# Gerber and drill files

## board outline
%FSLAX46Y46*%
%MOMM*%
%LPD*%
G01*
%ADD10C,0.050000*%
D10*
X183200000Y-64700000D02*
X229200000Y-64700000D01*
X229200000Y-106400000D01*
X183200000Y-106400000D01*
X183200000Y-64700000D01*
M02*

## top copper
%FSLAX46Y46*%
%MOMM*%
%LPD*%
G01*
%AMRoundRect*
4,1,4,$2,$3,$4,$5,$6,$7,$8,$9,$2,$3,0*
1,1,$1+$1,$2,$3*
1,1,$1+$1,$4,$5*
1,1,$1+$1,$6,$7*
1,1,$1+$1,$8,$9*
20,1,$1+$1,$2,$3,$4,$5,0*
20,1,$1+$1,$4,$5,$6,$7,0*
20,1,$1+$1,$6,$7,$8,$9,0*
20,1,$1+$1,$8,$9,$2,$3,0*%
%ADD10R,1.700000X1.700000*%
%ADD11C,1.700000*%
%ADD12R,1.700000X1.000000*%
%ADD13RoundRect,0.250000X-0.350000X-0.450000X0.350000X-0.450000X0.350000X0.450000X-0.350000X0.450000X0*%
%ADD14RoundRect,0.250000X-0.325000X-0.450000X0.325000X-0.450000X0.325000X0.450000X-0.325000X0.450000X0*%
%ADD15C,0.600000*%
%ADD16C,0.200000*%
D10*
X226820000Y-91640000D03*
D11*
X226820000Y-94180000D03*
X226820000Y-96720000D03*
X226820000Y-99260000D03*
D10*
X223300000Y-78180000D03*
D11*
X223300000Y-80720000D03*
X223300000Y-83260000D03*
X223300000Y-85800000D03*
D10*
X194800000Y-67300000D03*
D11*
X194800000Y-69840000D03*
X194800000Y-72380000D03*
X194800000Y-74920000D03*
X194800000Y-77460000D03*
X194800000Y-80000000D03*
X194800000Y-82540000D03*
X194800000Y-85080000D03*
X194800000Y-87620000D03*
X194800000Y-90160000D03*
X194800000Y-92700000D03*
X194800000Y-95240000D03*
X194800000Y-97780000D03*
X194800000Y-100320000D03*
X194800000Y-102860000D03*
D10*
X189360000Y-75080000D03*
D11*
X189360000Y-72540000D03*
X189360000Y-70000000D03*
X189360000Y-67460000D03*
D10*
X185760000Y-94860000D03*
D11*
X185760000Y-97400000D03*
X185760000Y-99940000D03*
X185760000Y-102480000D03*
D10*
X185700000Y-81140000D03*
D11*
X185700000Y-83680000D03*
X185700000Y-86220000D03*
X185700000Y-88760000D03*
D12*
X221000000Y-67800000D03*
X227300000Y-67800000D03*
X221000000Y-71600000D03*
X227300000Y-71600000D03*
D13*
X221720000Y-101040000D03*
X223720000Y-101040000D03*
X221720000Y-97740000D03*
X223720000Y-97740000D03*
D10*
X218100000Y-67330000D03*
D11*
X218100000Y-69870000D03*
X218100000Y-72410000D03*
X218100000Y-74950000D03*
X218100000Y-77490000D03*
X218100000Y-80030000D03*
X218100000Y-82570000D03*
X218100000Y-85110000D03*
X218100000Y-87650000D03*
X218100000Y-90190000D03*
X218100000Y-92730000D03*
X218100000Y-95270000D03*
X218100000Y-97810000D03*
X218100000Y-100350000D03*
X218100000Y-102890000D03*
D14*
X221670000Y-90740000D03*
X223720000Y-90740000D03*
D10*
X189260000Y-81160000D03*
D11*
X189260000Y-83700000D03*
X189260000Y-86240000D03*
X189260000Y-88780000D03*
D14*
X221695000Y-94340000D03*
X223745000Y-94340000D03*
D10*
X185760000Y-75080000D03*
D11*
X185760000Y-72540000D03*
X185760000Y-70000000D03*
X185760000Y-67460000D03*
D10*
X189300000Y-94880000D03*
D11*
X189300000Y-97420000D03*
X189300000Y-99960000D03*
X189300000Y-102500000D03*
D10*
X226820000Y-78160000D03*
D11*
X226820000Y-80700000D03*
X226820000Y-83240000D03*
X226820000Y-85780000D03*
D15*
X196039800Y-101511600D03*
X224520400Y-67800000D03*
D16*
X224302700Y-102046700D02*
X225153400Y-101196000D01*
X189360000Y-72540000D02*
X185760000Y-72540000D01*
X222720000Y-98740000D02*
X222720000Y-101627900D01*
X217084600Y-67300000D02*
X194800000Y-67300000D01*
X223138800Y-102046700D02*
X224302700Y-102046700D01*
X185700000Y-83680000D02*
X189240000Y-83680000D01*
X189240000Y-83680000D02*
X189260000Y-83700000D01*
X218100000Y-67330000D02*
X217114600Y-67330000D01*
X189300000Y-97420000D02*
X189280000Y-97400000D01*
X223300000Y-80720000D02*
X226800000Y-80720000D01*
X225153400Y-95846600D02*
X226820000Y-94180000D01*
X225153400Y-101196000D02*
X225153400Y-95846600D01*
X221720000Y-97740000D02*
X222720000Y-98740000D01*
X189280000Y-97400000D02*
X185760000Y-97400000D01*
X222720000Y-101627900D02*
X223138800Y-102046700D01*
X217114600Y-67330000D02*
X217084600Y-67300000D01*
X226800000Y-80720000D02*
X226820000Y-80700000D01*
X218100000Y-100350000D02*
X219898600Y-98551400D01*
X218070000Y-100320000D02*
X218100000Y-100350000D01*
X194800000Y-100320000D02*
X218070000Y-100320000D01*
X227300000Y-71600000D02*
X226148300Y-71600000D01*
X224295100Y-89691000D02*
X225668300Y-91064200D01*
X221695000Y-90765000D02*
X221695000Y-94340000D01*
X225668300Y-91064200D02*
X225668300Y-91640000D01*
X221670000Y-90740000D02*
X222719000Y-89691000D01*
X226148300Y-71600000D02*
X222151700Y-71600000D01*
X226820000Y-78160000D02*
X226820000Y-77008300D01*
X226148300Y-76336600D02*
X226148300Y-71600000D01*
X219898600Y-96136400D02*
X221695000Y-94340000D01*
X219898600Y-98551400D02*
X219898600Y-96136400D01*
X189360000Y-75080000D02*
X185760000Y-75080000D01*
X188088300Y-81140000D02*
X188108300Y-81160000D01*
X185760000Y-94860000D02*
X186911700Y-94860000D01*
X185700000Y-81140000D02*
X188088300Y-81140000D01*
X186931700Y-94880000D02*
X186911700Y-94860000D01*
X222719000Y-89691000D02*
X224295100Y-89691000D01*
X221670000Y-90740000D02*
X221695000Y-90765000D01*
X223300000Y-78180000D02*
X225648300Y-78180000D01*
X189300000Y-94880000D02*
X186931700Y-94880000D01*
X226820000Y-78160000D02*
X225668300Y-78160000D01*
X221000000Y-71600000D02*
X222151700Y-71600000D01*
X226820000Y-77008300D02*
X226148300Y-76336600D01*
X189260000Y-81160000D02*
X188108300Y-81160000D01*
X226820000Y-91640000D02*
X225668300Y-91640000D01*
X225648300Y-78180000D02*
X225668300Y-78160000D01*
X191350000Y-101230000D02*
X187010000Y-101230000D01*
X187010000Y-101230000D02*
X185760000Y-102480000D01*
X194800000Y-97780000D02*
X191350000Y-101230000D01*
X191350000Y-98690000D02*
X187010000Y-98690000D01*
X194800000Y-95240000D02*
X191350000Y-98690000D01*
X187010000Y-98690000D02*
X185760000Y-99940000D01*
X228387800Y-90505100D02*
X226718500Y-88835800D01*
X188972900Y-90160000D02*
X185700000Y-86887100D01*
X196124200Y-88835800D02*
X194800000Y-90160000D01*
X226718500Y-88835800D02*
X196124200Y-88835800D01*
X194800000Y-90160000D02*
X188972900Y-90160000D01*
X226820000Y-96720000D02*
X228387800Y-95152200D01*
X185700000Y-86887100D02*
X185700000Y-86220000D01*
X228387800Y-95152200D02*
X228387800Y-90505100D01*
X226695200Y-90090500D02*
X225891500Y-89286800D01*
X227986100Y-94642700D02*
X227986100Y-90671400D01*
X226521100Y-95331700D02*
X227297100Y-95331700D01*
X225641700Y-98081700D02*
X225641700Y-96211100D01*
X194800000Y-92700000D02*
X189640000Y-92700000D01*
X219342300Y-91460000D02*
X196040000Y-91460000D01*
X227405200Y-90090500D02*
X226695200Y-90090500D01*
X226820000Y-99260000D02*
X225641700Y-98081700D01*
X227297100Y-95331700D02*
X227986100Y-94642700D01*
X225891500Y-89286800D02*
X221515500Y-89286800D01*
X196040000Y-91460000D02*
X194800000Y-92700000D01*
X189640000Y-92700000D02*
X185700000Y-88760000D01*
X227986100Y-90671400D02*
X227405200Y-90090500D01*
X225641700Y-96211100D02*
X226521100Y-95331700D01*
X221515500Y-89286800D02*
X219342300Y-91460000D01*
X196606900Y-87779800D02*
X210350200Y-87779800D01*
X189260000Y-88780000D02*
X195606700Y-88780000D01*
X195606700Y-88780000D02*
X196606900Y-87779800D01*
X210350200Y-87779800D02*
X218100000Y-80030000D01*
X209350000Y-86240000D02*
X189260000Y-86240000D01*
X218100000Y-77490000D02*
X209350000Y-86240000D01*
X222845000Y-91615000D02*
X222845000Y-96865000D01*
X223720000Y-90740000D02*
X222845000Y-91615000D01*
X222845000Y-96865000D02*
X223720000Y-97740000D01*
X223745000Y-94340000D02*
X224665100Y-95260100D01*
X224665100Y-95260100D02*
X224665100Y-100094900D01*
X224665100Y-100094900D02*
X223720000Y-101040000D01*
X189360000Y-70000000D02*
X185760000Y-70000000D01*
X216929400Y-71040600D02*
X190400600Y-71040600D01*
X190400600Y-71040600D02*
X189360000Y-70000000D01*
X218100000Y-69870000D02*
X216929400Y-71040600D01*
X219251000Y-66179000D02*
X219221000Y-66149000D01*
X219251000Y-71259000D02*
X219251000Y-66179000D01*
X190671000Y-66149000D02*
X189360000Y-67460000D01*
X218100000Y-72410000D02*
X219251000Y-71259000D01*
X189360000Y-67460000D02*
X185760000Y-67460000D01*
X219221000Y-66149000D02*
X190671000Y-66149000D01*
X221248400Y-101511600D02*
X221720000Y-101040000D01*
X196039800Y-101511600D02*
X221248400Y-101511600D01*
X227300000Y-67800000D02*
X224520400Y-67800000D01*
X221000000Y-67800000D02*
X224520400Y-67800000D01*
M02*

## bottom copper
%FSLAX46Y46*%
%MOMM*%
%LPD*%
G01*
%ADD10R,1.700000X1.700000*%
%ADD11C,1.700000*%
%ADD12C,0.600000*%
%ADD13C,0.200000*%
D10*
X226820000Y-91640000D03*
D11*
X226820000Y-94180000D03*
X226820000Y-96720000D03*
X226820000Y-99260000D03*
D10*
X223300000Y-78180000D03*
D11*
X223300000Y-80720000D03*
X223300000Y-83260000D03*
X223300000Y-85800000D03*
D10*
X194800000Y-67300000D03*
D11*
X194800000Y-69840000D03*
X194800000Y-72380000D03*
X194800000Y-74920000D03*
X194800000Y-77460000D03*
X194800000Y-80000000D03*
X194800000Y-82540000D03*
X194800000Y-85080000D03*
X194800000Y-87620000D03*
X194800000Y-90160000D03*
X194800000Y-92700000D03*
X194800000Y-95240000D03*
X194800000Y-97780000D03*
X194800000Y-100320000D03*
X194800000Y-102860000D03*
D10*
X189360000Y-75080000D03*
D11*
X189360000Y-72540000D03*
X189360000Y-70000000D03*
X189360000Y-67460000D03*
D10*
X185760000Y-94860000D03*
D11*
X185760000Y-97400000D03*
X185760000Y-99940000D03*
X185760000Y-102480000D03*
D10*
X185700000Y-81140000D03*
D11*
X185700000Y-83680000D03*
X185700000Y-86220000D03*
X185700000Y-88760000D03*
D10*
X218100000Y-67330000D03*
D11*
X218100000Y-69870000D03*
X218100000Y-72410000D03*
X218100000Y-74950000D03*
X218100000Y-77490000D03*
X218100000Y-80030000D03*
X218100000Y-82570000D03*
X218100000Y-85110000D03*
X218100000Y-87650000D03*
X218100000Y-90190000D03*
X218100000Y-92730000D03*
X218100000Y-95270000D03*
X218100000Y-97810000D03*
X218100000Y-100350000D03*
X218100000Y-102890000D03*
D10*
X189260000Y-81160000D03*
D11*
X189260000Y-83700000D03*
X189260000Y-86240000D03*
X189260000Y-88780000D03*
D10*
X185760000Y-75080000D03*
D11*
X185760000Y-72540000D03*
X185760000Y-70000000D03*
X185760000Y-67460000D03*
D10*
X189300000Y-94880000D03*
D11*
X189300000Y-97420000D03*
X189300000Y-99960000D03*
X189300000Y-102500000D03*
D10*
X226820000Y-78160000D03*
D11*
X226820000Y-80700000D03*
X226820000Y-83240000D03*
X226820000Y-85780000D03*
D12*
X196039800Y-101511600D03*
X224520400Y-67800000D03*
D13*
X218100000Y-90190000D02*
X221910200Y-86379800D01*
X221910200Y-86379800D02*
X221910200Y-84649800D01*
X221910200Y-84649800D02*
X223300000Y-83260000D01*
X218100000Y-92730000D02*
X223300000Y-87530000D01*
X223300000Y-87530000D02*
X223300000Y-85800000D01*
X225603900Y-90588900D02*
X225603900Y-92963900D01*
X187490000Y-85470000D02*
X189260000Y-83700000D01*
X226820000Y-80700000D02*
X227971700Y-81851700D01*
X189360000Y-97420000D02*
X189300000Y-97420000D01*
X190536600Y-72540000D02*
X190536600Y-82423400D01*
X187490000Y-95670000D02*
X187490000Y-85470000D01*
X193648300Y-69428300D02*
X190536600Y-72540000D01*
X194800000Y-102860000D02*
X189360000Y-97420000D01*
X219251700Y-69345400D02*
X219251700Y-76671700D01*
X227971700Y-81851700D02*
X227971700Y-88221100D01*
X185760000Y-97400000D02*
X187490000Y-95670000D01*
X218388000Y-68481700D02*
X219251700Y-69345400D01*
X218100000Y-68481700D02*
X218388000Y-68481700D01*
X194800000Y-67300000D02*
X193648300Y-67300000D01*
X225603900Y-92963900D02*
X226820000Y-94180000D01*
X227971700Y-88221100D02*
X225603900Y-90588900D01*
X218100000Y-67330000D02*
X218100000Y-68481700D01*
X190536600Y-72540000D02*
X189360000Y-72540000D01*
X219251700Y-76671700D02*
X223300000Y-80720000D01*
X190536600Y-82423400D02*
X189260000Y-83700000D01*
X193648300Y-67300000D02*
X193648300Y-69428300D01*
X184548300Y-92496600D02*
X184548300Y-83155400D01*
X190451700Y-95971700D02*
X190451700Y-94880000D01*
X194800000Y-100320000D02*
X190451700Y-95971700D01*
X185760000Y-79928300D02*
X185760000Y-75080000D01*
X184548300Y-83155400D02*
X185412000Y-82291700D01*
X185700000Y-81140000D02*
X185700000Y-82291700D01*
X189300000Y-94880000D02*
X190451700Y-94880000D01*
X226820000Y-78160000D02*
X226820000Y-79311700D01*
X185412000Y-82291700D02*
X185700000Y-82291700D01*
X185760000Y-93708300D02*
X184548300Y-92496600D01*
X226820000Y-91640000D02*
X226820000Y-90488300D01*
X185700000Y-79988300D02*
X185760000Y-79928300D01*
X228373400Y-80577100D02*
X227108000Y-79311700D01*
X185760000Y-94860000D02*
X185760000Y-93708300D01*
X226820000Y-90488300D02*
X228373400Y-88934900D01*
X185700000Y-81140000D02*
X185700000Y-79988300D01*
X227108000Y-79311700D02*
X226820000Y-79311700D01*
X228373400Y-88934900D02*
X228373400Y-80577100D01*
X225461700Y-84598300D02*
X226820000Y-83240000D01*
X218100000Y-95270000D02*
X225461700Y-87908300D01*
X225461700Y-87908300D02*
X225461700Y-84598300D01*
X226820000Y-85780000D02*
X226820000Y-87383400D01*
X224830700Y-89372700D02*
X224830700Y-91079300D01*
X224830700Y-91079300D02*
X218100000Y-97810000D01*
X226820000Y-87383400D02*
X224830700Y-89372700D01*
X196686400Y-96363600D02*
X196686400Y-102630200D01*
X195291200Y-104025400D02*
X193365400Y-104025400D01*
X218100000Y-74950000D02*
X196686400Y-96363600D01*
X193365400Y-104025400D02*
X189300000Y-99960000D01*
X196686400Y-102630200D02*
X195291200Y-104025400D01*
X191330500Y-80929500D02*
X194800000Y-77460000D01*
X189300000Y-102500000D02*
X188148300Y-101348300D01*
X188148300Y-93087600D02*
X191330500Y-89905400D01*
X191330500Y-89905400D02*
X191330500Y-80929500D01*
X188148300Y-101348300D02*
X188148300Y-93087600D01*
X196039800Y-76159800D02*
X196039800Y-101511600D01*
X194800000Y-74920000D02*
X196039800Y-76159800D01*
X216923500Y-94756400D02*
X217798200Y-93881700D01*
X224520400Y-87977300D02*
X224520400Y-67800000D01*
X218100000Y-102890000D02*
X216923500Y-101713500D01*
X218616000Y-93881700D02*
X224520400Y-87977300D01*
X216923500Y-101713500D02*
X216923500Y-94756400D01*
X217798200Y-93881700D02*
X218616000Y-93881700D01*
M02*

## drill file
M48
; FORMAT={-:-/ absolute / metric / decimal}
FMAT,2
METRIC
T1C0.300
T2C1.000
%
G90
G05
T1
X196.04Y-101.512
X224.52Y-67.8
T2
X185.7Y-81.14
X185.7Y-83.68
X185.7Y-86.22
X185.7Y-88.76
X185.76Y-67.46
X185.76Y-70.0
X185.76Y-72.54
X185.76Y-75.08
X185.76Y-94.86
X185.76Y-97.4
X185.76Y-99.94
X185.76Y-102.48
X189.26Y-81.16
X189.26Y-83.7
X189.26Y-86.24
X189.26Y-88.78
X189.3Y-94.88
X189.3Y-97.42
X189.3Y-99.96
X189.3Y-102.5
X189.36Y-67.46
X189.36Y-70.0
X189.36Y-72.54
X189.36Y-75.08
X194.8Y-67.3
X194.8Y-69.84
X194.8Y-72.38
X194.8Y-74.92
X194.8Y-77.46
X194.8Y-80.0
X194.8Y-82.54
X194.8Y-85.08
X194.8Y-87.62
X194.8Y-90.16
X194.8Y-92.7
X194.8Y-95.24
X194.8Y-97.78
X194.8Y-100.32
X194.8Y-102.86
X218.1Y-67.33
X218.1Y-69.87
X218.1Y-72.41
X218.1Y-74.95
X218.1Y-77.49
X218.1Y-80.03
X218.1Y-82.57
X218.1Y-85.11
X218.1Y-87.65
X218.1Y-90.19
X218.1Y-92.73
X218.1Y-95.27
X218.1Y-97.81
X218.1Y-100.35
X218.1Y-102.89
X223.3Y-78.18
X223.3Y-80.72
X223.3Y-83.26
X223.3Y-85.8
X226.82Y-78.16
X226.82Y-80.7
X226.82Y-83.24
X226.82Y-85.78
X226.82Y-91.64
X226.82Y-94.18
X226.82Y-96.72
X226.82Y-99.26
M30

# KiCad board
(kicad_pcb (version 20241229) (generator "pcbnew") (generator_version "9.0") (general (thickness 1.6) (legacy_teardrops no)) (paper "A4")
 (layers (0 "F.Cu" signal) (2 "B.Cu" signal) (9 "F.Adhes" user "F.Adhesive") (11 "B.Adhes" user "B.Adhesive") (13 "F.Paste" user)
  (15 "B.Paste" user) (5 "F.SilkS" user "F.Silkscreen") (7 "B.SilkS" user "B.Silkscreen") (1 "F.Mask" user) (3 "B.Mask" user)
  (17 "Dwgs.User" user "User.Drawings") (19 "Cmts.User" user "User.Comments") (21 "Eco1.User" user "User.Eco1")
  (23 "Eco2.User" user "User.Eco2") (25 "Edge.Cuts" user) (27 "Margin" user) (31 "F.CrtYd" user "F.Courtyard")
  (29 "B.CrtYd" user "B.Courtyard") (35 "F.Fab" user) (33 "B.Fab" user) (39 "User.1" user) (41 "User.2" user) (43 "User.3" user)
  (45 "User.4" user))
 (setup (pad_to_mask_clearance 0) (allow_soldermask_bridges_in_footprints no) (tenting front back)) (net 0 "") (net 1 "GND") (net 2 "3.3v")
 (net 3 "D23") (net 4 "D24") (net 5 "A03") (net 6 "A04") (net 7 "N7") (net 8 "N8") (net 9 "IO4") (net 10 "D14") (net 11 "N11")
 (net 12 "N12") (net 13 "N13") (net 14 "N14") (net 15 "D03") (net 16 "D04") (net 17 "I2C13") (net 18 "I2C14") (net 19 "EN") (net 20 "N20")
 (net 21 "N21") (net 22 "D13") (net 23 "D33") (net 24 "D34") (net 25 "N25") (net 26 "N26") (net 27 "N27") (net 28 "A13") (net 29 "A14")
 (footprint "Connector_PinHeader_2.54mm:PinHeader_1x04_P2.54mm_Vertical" (layer "F.Cu") (at 226.82 91.64)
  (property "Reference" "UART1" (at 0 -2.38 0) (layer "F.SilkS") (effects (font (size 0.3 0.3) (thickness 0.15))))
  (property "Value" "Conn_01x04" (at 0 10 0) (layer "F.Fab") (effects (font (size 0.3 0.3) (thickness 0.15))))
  (pad "1" thru_hole rect (at 0 0) (size 1.7 1.7) (drill 1) (layers "*.Cu" "*.Mask") (remove_unused_layers no) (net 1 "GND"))
  (pad "2" thru_hole circle (at 0 2.54) (size 1.7 1.7) (drill 1) (layers "*.Cu" "*.Mask") (remove_unused_layers no) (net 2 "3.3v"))
  (pad "3" thru_hole circle (at 0 5.08) (size 1.7 1.7) (drill 1) (layers "*.Cu" "*.Mask") (remove_unused_layers no) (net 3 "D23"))
  (pad "4" thru_hole circle (at 0 7.62) (size 1.7 1.7) (drill 1) (layers "*.Cu" "*.Mask") (remove_unused_layers no) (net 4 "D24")))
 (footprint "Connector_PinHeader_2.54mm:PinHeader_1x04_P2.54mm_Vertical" (layer "F.Cu") (at 223.3 78.18)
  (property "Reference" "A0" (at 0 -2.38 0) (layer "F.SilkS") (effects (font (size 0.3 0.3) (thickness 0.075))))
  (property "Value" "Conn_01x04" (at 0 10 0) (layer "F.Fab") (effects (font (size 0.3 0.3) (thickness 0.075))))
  (pad "1" thru_hole rect (at 0 0) (size 1.7 1.7) (drill 1) (layers "*.Cu" "*.Mask") (remove_unused_layers no) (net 1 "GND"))
  (pad "2" thru_hole circle (at 0 2.54) (size 1.7 1.7) (drill 1) (layers "*.Cu" "*.Mask") (remove_unused_layers no) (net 2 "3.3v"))
  (pad "3" thru_hole circle (at 0 5.08) (size 1.7 1.7) (drill 1) (layers "*.Cu" "*.Mask") (remove_unused_layers no) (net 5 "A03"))
  (pad "4" thru_hole circle (at 0 7.62) (size 1.7 1.7) (drill 1) (layers "*.Cu" "*.Mask") (remove_unused_layers no) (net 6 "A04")))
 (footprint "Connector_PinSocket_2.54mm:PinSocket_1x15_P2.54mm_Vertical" (layer "F.Cu") (at 194.8 67.3)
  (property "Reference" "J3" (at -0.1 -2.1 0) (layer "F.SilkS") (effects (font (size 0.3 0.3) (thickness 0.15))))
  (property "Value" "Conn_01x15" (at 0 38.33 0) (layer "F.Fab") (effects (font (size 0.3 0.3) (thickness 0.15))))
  (pad "1" thru_hole rect (at 0 0) (size 1.7 1.7) (drill 1) (layers "*.Cu" "*.Mask") (remove_unused_layers no) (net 2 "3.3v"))
  (pad "2" thru_hole circle (at 0 2.54) (size 1.7 1.7) (drill 1) (layers "*.Cu" "*.Mask") (remove_unused_layers no) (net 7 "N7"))
  (pad "3" thru_hole circle (at 0 5.08) (size 1.7 1.7) (drill 1) (layers "*.Cu" "*.Mask") (remove_unused_layers no) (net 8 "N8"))
  (pad "4" thru_hole circle (at 0 7.62) (size 1.7 1.7) (drill 1) (layers "*.Cu" "*.Mask") (remove_unused_layers no) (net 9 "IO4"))
  (pad "5" thru_hole circle (at 0 10.16) (size 1.7 1.7) (drill 1) (layers "*.Cu" "*.Mask") (remove_unused_layers no) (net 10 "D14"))
  (pad "6" thru_hole circle (at 0 12.7) (size 1.7 1.7) (drill 1) (layers "*.Cu" "*.Mask") (remove_unused_layers no) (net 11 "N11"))
  (pad "7" thru_hole circle (at 0 15.24) (size 1.7 1.7) (drill 1) (layers "*.Cu" "*.Mask") (remove_unused_layers no) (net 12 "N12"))
  (pad "8" thru_hole circle (at 0 17.78) (size 1.7 1.7) (drill 1) (layers "*.Cu" "*.Mask") (remove_unused_layers no) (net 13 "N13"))
  (pad "9" thru_hole circle (at 0 20.32) (size 1.7 1.7) (drill 1) (layers "*.Cu" "*.Mask") (remove_unused_layers no) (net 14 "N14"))
  (pad "10" thru_hole circle (at 0 22.86) (size 1.7 1.7) (drill 1) (layers "*.Cu" "*.Mask") (remove_unused_layers no) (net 3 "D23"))
  (pad "11" thru_hole circle (at 0 25.4) (size 1.7 1.7) (drill 1) (layers "*.Cu" "*.Mask") (remove_unused_layers no) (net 4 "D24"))
  (pad "12" thru_hole circle (at 0 27.94) (size 1.7 1.7) (drill 1) (layers "*.Cu" "*.Mask") (remove_unused_layers no) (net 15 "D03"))
  (pad "13" thru_hole circle (at 0 30.48) (size 1.7 1.7) (drill 1) (layers "*.Cu" "*.Mask") (remove_unused_layers no) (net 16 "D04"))
  (pad "14" thru_hole circle (at 0 33.02) (size 1.7 1.7) (drill 1) (layers "*.Cu" "*.Mask") (remove_unused_layers no) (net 1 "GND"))
  (pad "15" thru_hole circle (at 0 35.56) (size 1.7 1.7) (drill 1) (layers "*.Cu" "*.Mask") (remove_unused_layers no) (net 2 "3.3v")))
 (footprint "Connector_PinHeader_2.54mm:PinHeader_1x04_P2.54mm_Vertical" (layer "F.Cu") (at 189.36 75.08 180)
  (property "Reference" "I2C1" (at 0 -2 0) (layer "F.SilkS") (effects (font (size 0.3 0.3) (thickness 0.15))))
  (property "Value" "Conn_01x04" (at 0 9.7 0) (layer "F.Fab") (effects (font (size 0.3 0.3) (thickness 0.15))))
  (pad "1" thru_hole rect (at 0 0 180) (size 1.7 1.7) (drill 1) (layers "*.Cu" "*.Mask") (remove_unused_layers no) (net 1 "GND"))
  (pad "2" thru_hole circle (at 0 2.54 180) (size 1.7 1.7) (drill 1) (layers "*.Cu" "*.Mask") (remove_unused_layers no) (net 2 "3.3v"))
  (pad "3" thru_hole circle (at 0 5.08 180) (size 1.7 1.7) (drill 1) (layers "*.Cu" "*.Mask") (remove_unused_layers no) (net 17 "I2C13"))
  (pad "4" thru_hole circle (at 0 7.62 180) (size 1.7 1.7) (drill 1) (layers "*.Cu" "*.Mask") (remove_unused_layers no) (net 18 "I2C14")))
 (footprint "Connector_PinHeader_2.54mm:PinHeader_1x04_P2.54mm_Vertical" (layer "F.Cu") (at 185.76 94.86)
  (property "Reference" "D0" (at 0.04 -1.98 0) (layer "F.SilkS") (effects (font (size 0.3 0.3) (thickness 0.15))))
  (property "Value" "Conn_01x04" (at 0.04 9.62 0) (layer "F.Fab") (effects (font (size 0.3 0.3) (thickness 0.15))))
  (pad "1" thru_hole rect (at 0 0) (size 1.7 1.7) (drill 1) (layers "*.Cu" "*.Mask") (remove_unused_layers no) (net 1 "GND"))
  (pad "2" thru_hole circle (at 0 2.54) (size 1.7 1.7) (drill 1) (layers "*.Cu" "*.Mask") (remove_unused_layers no) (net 2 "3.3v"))
  (pad "3" thru_hole circle (at 0 5.08) (size 1.7 1.7) (drill 1) (layers "*.Cu" "*.Mask") (remove_unused_layers no) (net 15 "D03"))
  (pad "4" thru_hole circle (at 0 7.62) (size 1.7 1.7) (drill 1) (layers "*.Cu" "*.Mask") (remove_unused_layers no) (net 16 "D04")))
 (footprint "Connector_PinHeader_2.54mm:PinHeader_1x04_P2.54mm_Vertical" (layer "F.Cu") (at 185.7 81.14)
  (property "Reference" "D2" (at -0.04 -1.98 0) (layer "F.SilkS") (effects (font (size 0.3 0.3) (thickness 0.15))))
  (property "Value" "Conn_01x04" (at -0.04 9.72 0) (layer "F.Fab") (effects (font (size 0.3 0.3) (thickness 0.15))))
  (pad "1" thru_hole rect (at 0 0) (size 1.7 1.7) (drill 1) (layers "*.Cu" "*.Mask") (remove_unused_layers no) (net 1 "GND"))
  (pad "2" thru_hole circle (at 0 2.54) (size 1.7 1.7) (drill 1) (layers "*.Cu" "*.Mask") (remove_unused_layers no) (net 2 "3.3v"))
  (pad "3" thru_hole circle (at 0 5.08) (size 1.7 1.7) (drill 1) (layers "*.Cu" "*.Mask") (remove_unused_layers no) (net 3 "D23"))
  (pad "4" thru_hole circle (at 0 7.62) (size 1.7 1.7) (drill 1) (layers "*.Cu" "*.Mask") (remove_unused_layers no) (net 4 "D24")))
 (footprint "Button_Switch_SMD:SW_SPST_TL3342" (layer "F.Cu") (at 224.15 69.7)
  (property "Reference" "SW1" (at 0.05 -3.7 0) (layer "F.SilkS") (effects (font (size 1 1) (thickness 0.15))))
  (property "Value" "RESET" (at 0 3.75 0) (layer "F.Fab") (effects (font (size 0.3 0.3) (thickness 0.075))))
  (pad "1" smd rect (at -3.15 -1.9) (size 1.7 1) (layers "F.Cu" "F.Mask" "F.Paste") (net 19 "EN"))
  (pad "1" smd rect (at 3.15 -1.9) (size 1.7 1) (layers "F.Cu" "F.Mask" "F.Paste") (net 19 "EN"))
  (pad "2" smd rect (at -3.15 1.9) (size 1.7 1) (layers "F.Cu" "F.Mask" "F.Paste") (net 1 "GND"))
  (pad "2" smd rect (at 3.15 1.9) (size 1.7 1) (layers "F.Cu" "F.Mask" "F.Paste") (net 1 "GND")))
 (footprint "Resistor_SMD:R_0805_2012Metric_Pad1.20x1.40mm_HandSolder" (layer "F.Cu") (at 222.72 101.04)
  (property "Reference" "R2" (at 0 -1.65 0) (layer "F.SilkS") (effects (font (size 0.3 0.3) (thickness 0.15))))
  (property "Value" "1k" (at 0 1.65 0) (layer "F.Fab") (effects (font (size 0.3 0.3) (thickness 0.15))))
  (pad "1" smd roundrect (at -1 0) (size 1.2 1.4) (layers "F.Cu" "F.Mask" "F.Paste") (roundrect_rratio 0.208333) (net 9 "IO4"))
  (pad "2" smd roundrect (at 1 0) (size 1.2 1.4) (layers "F.Cu" "F.Mask" "F.Paste") (roundrect_rratio 0.208333) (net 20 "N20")))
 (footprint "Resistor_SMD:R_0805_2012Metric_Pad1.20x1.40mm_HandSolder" (layer "F.Cu") (at 222.72 97.74)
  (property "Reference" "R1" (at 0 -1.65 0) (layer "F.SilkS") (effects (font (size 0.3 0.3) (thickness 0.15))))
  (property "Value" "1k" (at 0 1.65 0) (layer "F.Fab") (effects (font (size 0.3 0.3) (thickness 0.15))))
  (pad "1" smd roundrect (at -1 0) (size 1.2 1.4) (layers "F.Cu" "F.Mask" "F.Paste") (roundrect_rratio 0.208333) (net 2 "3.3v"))
  (pad "2" smd roundrect (at 1 0) (size 1.2 1.4) (layers "F.Cu" "F.Mask" "F.Paste") (roundrect_rratio 0.208333) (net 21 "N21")))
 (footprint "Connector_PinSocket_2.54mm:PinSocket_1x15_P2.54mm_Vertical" (layer "F.Cu") (at 218.1 67.33)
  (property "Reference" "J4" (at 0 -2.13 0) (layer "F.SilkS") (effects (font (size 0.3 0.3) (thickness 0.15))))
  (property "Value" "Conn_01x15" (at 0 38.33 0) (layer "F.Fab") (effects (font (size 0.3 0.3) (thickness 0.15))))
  (pad "1" thru_hole rect (at 0 0) (size 1.7 1.7) (drill 1) (layers "*.Cu" "*.Mask") (remove_unused_layers no) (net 2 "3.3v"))
  (pad "2" thru_hole circle (at 0 2.54) (size 1.7 1.7) (drill 1) (layers "*.Cu" "*.Mask") (remove_unused_layers no) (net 17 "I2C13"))
  (pad "3" thru_hole circle (at 0 5.08) (size 1.7 1.7) (drill 1) (layers "*.Cu" "*.Mask") (remove_unused_layers no) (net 18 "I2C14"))
  (pad "4" thru_hole circle (at 0 7.62) (size 1.7 1.7) (drill 1) (layers "*.Cu" "*.Mask") (remove_unused_layers no) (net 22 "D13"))
  (pad "5" thru_hole circle (at 0 10.16) (size 1.7 1.7) (drill 1) (layers "*.Cu" "*.Mask") (remove_unused_layers no) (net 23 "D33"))
  (pad "6" thru_hole circle (at 0 12.7) (size 1.7 1.7) (drill 1) (layers "*.Cu" "*.Mask") (remove_unused_layers no) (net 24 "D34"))
  (pad "7" thru_hole circle (at 0 15.24) (size 1.7 1.7) (drill 1) (layers "*.Cu" "*.Mask") (remove_unused_layers no) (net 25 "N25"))
  (pad "8" thru_hole circle (at 0 17.78) (size 1.7 1.7) (drill 1) (layers "*.Cu" "*.Mask") (remove_unused_layers no) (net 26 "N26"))
  (pad "9" thru_hole circle (at 0 20.32) (size 1.7 1.7) (drill 1) (layers "*.Cu" "*.Mask") (remove_unused_layers no) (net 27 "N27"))
  (pad "10" thru_hole circle (at 0 22.86) (size 1.7 1.7) (drill 1) (layers "*.Cu" "*.Mask") (remove_unused_layers no) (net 5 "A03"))
  (pad "11" thru_hole circle (at 0 25.4) (size 1.7 1.7) (drill 1) (layers "*.Cu" "*.Mask") (remove_unused_layers no) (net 6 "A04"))
  (pad "12" thru_hole circle (at 0 27.94) (size 1.7 1.7) (drill 1) (layers "*.Cu" "*.Mask") (remove_unused_layers no) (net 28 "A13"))
  (pad "13" thru_hole circle (at 0 30.48) (size 1.7 1.7) (drill 1) (layers "*.Cu" "*.Mask") (remove_unused_layers no) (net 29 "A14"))
  (pad "14" thru_hole circle (at 0 33.02) (size 1.7 1.7) (drill 1) (layers "*.Cu" "*.Mask") (remove_unused_layers no) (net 1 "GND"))
  (pad "15" thru_hole circle (at 0 35.56) (size 1.7 1.7) (drill 1) (layers "*.Cu" "*.Mask") (remove_unused_layers no) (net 19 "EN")))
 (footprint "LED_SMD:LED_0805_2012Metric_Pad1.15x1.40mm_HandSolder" (layer "F.Cu") (at 222.695 90.74)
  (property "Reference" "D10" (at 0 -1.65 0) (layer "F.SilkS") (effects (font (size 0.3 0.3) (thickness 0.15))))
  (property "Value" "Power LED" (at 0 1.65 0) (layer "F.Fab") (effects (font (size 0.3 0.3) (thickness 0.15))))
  (pad "1" smd roundrect (at -1.025 0) (size 1.15 1.4) (layers "F.Cu" "F.Mask" "F.Paste") (roundrect_rratio 0.217391) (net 1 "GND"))
  (pad "2" smd roundrect (at 1.025 0) (size 1.15 1.4) (layers "F.Cu" "F.Mask" "F.Paste") (roundrect_rratio 0.217391) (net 21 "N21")))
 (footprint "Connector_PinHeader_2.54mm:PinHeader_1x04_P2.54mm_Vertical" (layer "F.Cu") (at 189.26 81.16)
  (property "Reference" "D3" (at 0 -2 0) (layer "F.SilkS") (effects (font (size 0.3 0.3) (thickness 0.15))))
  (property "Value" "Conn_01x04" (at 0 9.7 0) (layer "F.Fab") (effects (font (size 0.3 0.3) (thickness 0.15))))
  (pad "1" thru_hole rect (at 0 0) (size 1.7 1.7) (drill 1) (layers "*.Cu" "*.Mask") (remove_unused_layers no) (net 1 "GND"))
  (pad "2" thru_hole circle (at 0 2.54) (size 1.7 1.7) (drill 1) (layers "*.Cu" "*.Mask") (remove_unused_layers no) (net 2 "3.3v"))
  (pad "3" thru_hole circle (at 0 5.08) (size 1.7 1.7) (drill 1) (layers "*.Cu" "*.Mask") (remove_unused_layers no) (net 23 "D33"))
  (pad "4" thru_hole circle (at 0 7.62) (size 1.7 1.7) (drill 1) (layers "*.Cu" "*.Mask") (remove_unused_layers no) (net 24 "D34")))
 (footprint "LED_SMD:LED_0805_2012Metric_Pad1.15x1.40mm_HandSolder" (layer "F.Cu") (at 222.72 94.34)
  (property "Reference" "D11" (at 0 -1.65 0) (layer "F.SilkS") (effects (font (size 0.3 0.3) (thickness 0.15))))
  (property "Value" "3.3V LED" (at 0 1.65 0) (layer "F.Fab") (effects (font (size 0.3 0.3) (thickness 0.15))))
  (pad "1" smd roundrect (at -1.025 0) (size 1.15 1.4) (layers "F.Cu" "F.Mask" "F.Paste") (roundrect_rratio 0.217391) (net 1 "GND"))
  (pad "2" smd roundrect (at 1.025 0) (size 1.15 1.4) (layers "F.Cu" "F.Mask" "F.Paste") (roundrect_rratio 0.217391) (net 20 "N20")))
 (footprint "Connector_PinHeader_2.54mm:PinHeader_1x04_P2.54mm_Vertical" (layer "F.Cu") (at 185.76 75.08 180)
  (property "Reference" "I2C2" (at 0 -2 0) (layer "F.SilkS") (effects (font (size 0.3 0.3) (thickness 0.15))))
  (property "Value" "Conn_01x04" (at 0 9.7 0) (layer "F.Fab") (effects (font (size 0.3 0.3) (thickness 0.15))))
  (pad "1" thru_hole rect (at 0 0 180) (size 1.7 1.7) (drill 1) (layers "*.Cu" "*.Mask") (remove_unused_layers no) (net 1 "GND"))
  (pad "2" thru_hole circle (at 0 2.54 180) (size 1.7 1.7) (drill 1) (layers "*.Cu" "*.Mask") (remove_unused_layers no) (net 2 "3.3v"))
  (pad "3" thru_hole circle (at 0 5.08 180) (size 1.7 1.7) (drill 1) (layers "*.Cu" "*.Mask") (remove_unused_layers no) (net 17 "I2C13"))
  (pad "4" thru_hole circle (at 0 7.62 180) (size 1.7 1.7) (drill 1) (layers "*.Cu" "*.Mask") (remove_unused_layers no) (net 18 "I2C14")))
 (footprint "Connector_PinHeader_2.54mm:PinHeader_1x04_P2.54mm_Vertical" (layer "F.Cu") (at 189.3 94.88)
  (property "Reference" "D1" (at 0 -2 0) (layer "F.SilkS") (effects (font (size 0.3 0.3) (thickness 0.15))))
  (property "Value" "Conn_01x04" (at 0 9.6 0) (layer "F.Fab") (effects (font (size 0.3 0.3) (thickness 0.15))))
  (pad "1" thru_hole rect (at 0 0) (size 1.7 1.7) (drill 1) (layers "*.Cu" "*.Mask") (remove_unused_layers no) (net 1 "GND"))
  (pad "2" thru_hole circle (at 0 2.54) (size 1.7 1.7) (drill 1) (layers "*.Cu" "*.Mask") (remove_unused_layers no) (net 2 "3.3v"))
  (pad "3" thru_hole circle (at 0 5.08) (size 1.7 1.7) (drill 1) (layers "*.Cu" "*.Mask") (remove_unused_layers no) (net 22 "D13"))
  (pad "4" thru_hole circle (at 0 7.62) (size 1.7 1.7) (drill 1) (layers "*.Cu" "*.Mask") (remove_unused_layers no) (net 10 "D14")))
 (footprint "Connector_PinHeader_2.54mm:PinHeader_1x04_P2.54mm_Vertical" (layer "F.Cu") (at 226.82 78.16)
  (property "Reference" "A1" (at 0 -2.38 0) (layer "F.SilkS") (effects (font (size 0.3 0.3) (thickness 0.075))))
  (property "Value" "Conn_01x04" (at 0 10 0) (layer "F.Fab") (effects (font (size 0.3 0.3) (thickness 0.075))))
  (pad "1" thru_hole rect (at 0 0) (size 1.7 1.7) (drill 1) (layers "*.Cu" "*.Mask") (remove_unused_layers no) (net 1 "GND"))
  (pad "2" thru_hole circle (at 0 2.54) (size 1.7 1.7) (drill 1) (layers "*.Cu" "*.Mask") (remove_unused_layers no) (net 2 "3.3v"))
  (pad "3" thru_hole circle (at 0 5.08) (size 1.7 1.7) (drill 1) (layers "*.Cu" "*.Mask") (remove_unused_layers no) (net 28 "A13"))
  (pad "4" thru_hole circle (at 0 7.62) (size 1.7 1.7) (drill 1) (layers "*.Cu" "*.Mask") (remove_unused_layers no) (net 29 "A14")))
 (gr_rect (start 183.2 64.7) (end 229.2 106.4) (stroke (width 0.05) (type default)) (fill no) (layer "Edge.Cuts"))
 (segment (start 218.1 90.19) (end 221.9102 86.3798) (width 0.2) (layer "B.Cu") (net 5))
 (segment (start 221.9102 86.3798) (end 221.9102 84.6498) (width 0.2) (layer "B.Cu") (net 5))
 (segment (start 221.9102 84.6498) (end 223.3 83.26) (width 0.2) (layer "B.Cu") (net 5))
 (segment (start 218.1 92.73) (end 223.3 87.53) (width 0.2) (layer "B.Cu") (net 6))
 (segment (start 223.3 87.53) (end 223.3 85.8) (width 0.2) (layer "B.Cu") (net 6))
 (segment (start 224.3027 102.0467) (end 225.1534 101.196) (width 0.2) (layer "F.Cu") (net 2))
 (segment (start 189.36 72.54) (end 185.76 72.54) (width 0.2) (layer "F.Cu") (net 2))
 (segment (start 222.72 98.74) (end 222.72 101.6279) (width 0.2) (layer "F.Cu") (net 2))
 (segment (start 217.0846 67.3) (end 194.8 67.3) (width 0.2) (layer "F.Cu") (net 2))
 (segment (start 223.1388 102.0467) (end 224.3027 102.0467) (width 0.2) (layer "F.Cu") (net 2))
 (segment (start 185.7 83.68) (end 189.24 83.68) (width 0.2) (layer "F.Cu") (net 2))
 (segment (start 189.24 83.68) (end 189.26 83.7) (width 0.2) (layer "F.Cu") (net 2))
 (segment (start 218.1 67.33) (end 217.1146 67.33) (width 0.2) (layer "F.Cu") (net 2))
 (segment (start 189.3 97.42) (end 189.28 97.4) (width 0.2) (layer "F.Cu") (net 2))
 (segment (start 223.3 80.72) (end 226.8 80.72) (width 0.2) (layer "F.Cu") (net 2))
 (segment (start 225.1534 95.8466) (end 226.82 94.18) (width 0.2) (layer "F.Cu") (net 2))
 (segment (start 225.1534 101.196) (end 225.1534 95.8466) (width 0.2) (layer "F.Cu") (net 2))
 (segment (start 221.72 97.74) (end 222.72 98.74) (width 0.2) (layer "F.Cu") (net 2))
 (segment (start 189.28 97.4) (end 185.76 97.4) (width 0.2) (layer "F.Cu") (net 2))
 (segment (start 222.72 101.6279) (end 223.1388 102.0467) (width 0.2) (layer "F.Cu") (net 2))
 (segment (start 217.1146 67.33) (end 217.0846 67.3) (width 0.2) (layer "F.Cu") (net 2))
 (segment (start 226.8 80.72) (end 226.82 80.7) (width 0.2) (layer "F.Cu") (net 2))
 (segment (start 225.6039 90.5889) (end 225.6039 92.9639) (width 0.2) (layer "B.Cu") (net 2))
 (segment (start 187.49 85.47) (end 189.26 83.7) (width 0.2) (layer "B.Cu") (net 2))
 (segment (start 226.82 80.7) (end 227.9717 81.8517) (width 0.2) (layer "B.Cu") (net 2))
 (segment (start 189.36 97.42) (end 189.3 97.42) (width 0.2) (layer "B.Cu") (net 2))
 (segment (start 190.5366 72.54) (end 190.5366 82.4234) (width 0.2) (layer "B.Cu") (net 2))
 (segment (start 187.49 95.67) (end 187.49 85.47) (width 0.2) (layer "B.Cu") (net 2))
 (segment (start 193.6483 69.4283) (end 190.5366 72.54) (width 0.2) (layer "B.Cu") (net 2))
 (segment (start 194.8 102.86) (end 189.36 97.42) (width 0.2) (layer "B.Cu") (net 2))
 (segment (start 219.2517 69.3454) (end 219.2517 76.6717) (width 0.2) (layer "B.Cu") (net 2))
 (segment (start 227.9717 81.8517) (end 227.9717 88.2211) (width 0.2) (layer "B.Cu") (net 2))
 (segment (start 185.76 97.4) (end 187.49 95.67) (width 0.2) (layer "B.Cu") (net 2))
 (segment (start 218.388 68.4817) (end 219.2517 69.3454) (width 0.2) (layer "B.Cu") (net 2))
 (segment (start 218.1 68.4817) (end 218.388 68.4817) (width 0.2) (layer "B.Cu") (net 2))
 (segment (start 194.8 67.3) (end 193.6483 67.3) (width 0.2) (layer "B.Cu") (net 2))
 (segment (start 225.6039 92.9639) (end 226.82 94.18) (width 0.2) (layer "B.Cu") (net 2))
 (segment (start 227.9717 88.2211) (end 225.6039 90.5889) (width 0.2) (layer "B.Cu") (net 2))
 (segment (start 218.1 67.33) (end 218.1 68.4817) (width 0.2) (layer "B.Cu") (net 2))
 (segment (start 190.5366 72.54) (end 189.36 72.54) (width 0.2) (layer "B.Cu") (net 2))
 (segment (start 219.2517 76.6717) (end 223.3 80.72) (width 0.2) (layer "B.Cu") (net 2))
 (segment (start 190.5366 82.4234) (end 189.26 83.7) (width 0.2) (layer "B.Cu") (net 2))
 (segment (start 193.6483 67.3) (end 193.6483 69.4283) (width 0.2) (layer "B.Cu") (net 2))
 (segment (start 218.1 100.35) (end 219.8986 98.5514) (width 0.2) (layer "F.Cu") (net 1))
 (segment (start 218.07 100.32) (end 218.1 100.35) (width 0.2) (layer "F.Cu") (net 1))
 (segment (start 194.8 100.32) (end 218.07 100.32) (width 0.2) (layer "F.Cu") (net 1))
 (segment (start 227.3 71.6) (end 226.1483 71.6) (width 0.2) (layer "F.Cu") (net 1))
 (segment (start 224.2951 89.691) (end 225.6683 91.0642) (width 0.2) (layer "F.Cu") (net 1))
 (segment (start 221.695 90.765) (end 221.695 94.34) (width 0.2) (layer "F.Cu") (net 1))
 (segment (start 225.6683 91.0642) (end 225.6683 91.64) (width 0.2) (layer "F.Cu") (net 1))
 (segment (start 221.67 90.74) (end 222.719 89.691) (width 0.2) (layer "F.Cu") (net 1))
 (segment (start 226.1483 71.6) (end 222.1517 71.6) (width 0.2) (layer "F.Cu") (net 1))
 (segment (start 226.82 78.16) (end 226.82 77.0083) (width 0.2) (layer "F.Cu") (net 1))
 (segment (start 226.1483 76.3366) (end 226.1483 71.6) (width 0.2) (layer "F.Cu") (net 1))
 (segment (start 219.8986 96.1364) (end 221.695 94.34) (width 0.2) (layer "F.Cu") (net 1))
 (segment (start 219.8986 98.5514) (end 219.8986 96.1364) (width 0.2) (layer "F.Cu") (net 1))
 (segment (start 189.36 75.08) (end 185.76 75.08) (width 0.2) (layer "F.Cu") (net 1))
 (segment (start 188.0883 81.14) (end 188.1083 81.16) (width 0.2) (layer "F.Cu") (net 1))
 (segment (start 185.76 94.86) (end 186.9117 94.86) (width 0.2) (layer "F.Cu") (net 1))
 (segment (start 185.7 81.14) (end 188.0883 81.14) (width 0.2) (layer "F.Cu") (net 1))
 (segment (start 186.9317 94.88) (end 186.9117 94.86) (width 0.2) (layer "F.Cu") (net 1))
 (segment (start 222.719 89.691) (end 224.2951 89.691) (width 0.2) (layer "F.Cu") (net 1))
 (segment (start 221.67 90.74) (end 221.695 90.765) (width 0.2) (layer "F.Cu") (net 1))
 (segment (start 223.3 78.18) (end 225.6483 78.18) (width 0.2) (layer "F.Cu") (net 1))
 (segment (start 189.3 94.88) (end 186.9317 94.88) (width 0.2) (layer "F.Cu") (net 1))
 (segment (start 226.82 78.16) (end 225.6683 78.16) (width 0.2) (layer "F.Cu") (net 1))
 (segment (start 221 71.6) (end 222.1517 71.6) (width 0.2) (layer "F.Cu") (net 1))
 (segment (start 226.82 77.0083) (end 226.1483 76.3366) (width 0.2) (layer "F.Cu") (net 1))
 (segment (start 189.26 81.16) (end 188.1083 81.16) (width 0.2) (layer "F.Cu") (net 1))
 (segment (start 226.82 91.64) (end 225.6683 91.64) (width 0.2) (layer "F.Cu") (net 1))
 (segment (start 225.6483 78.18) (end 225.6683 78.16) (width 0.2) (layer "F.Cu") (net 1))
 (segment (start 184.5483 92.4966) (end 184.5483 83.1554) (width 0.2) (layer "B.Cu") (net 1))
 (segment (start 190.4517 95.9717) (end 190.4517 94.88) (width 0.2) (layer "B.Cu") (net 1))
 (segment (start 194.8 100.32) (end 190.4517 95.9717) (width 0.2) (layer "B.Cu") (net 1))
 (segment (start 185.76 79.9283) (end 185.76 75.08) (width 0.2) (layer "B.Cu") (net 1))
 (segment (start 184.5483 83.1554) (end 185.412 82.2917) (width 0.2) (layer "B.Cu") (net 1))
 (segment (start 185.7 81.14) (end 185.7 82.2917) (width 0.2) (layer "B.Cu") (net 1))
 (segment (start 189.3 94.88) (end 190.4517 94.88) (width 0.2) (layer "B.Cu") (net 1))
 (segment (start 226.82 78.16) (end 226.82 79.3117) (width 0.2) (layer "B.Cu") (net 1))
 (segment (start 185.412 82.2917) (end 185.7 82.2917) (width 0.2) (layer "B.Cu") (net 1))
 (segment (start 185.76 93.7083) (end 184.5483 92.4966) (width 0.2) (layer "B.Cu") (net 1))
 (segment (start 226.82 91.64) (end 226.82 90.4883) (width 0.2) (layer "B.Cu") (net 1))
 (segment (start 185.7 79.9883) (end 185.76 79.9283) (width 0.2) (layer "B.Cu") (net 1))
 (segment (start 228.3734 80.5771) (end 227.108 79.3117) (width 0.2) (layer "B.Cu") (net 1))
 (segment (start 185.76 94.86) (end 185.76 93.7083) (width 0.2) (layer "B.Cu") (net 1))
 (segment (start 226.82 90.4883) (end 228.3734 88.9349) (width 0.2) (layer "B.Cu") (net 1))
 (segment (start 185.7 81.14) (end 185.7 79.9883) (width 0.2) (layer "B.Cu") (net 1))
 (segment (start 227.108 79.3117) (end 226.82 79.3117) (width 0.2) (layer "B.Cu") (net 1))
 (segment (start 228.3734 88.9349) (end 228.3734 80.5771) (width 0.2) (layer "B.Cu") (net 1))
 (segment (start 225.4617 84.5983) (end 226.82 83.24) (width 0.2) (layer "B.Cu") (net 28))
 (segment (start 218.1 95.27) (end 225.4617 87.9083) (width 0.2) (layer "B.Cu") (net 28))
 (segment (start 225.4617 87.9083) (end 225.4617 84.5983) (width 0.2) (layer "B.Cu") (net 28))
 (segment (start 226.82 85.78) (end 226.82 87.3834) (width 0.2) (layer "B.Cu") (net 29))
 (segment (start 224.8307 89.3727) (end 224.8307 91.0793) (width 0.2) (layer "B.Cu") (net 29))
 (segment (start 224.8307 91.0793) (end 218.1 97.81) (width 0.2) (layer "B.Cu") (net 29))
 (segment (start 226.82 87.3834) (end 224.8307 89.3727) (width 0.2) (layer "B.Cu") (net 29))
 (segment (start 191.35 101.23) (end 187.01 101.23) (width 0.2) (layer "F.Cu") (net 16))
 (segment (start 187.01 101.23) (end 185.76 102.48) (width 0.2) (layer "F.Cu") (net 16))
 (segment (start 194.8 97.78) (end 191.35 101.23) (width 0.2) (layer "F.Cu") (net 16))
 (segment (start 191.35 98.69) (end 187.01 98.69) (width 0.2) (layer "F.Cu") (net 15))
 (segment (start 194.8 95.24) (end 191.35 98.69) (width 0.2) (layer "F.Cu") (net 15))
 (segment (start 187.01 98.69) (end 185.76 99.94) (width 0.2) (layer "F.Cu") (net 15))
 (segment (start 196.6864 96.3636) (end 196.6864 102.6302) (width 0.2) (layer "B.Cu") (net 22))
 (segment (start 195.2912 104.0254) (end 193.3654 104.0254) (width 0.2) (layer "B.Cu") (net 22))
 (segment (start 218.1 74.95) (end 196.6864 96.3636) (width 0.2) (layer "B.Cu") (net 22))
 (segment (start 193.3654 104.0254) (end 189.3 99.96) (width 0.2) (layer "B.Cu") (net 22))
 (segment (start 196.6864 102.6302) (end 195.2912 104.0254) (width 0.2) (layer "B.Cu") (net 22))
 (segment (start 191.3305 80.9295) (end 194.8 77.46) (width 0.2) (layer "B.Cu") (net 10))
 (segment (start 189.3 102.5) (end 188.1483 101.3483) (width 0.2) (layer "B.Cu") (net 10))
 (segment (start 188.1483 93.0876) (end 191.3305 89.9054) (width 0.2) (layer "B.Cu") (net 10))
 (segment (start 191.3305 89.9054) (end 191.3305 80.9295) (width 0.2) (layer "B.Cu") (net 10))
 (segment (start 188.1483 101.3483) (end 188.1483 93.0876) (width 0.2) (layer "B.Cu") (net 10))
 (segment (start 228.3878 90.5051) (end 226.7185 88.8358) (width 0.2) (layer "F.Cu") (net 3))
 (segment (start 188.9729 90.16) (end 185.7 86.8871) (width 0.2) (layer "F.Cu") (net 3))
 (segment (start 196.1242 88.8358) (end 194.8 90.16) (width 0.2) (layer "F.Cu") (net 3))
 (segment (start 226.7185 88.8358) (end 196.1242 88.8358) (width 0.2) (layer "F.Cu") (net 3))
 (segment (start 194.8 90.16) (end 188.9729 90.16) (width 0.2) (layer "F.Cu") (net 3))
 (segment (start 226.82 96.72) (end 228.3878 95.1522) (width 0.2) (layer "F.Cu") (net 3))
 (segment (start 185.7 86.8871) (end 185.7 86.22) (width 0.2) (layer "F.Cu") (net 3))
 (segment (start 228.3878 95.1522) (end 228.3878 90.5051) (width 0.2) (layer "F.Cu") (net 3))
 (segment (start 226.6952 90.0905) (end 225.8915 89.2868) (width 0.2) (layer "F.Cu") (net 4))
 (segment (start 227.9861 94.6427) (end 227.9861 90.6714) (width 0.2) (layer "F.Cu") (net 4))
 (segment (start 226.5211 95.3317) (end 227.2971 95.3317) (width 0.2) (layer "F.Cu") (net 4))
 (segment (start 225.6417 98.0817) (end 225.6417 96.2111) (width 0.2) (layer "F.Cu") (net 4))
 (segment (start 194.8 92.7) (end 189.64 92.7) (width 0.2) (layer "F.Cu") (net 4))
 (segment (start 219.3423 91.46) (end 196.04 91.46) (width 0.2) (layer "F.Cu") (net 4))
 (segment (start 227.4052 90.0905) (end 226.6952 90.0905) (width 0.2) (layer "F.Cu") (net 4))
 (segment (start 226.82 99.26) (end 225.6417 98.0817) (width 0.2) (layer "F.Cu") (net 4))
 (segment (start 227.2971 95.3317) (end 227.9861 94.6427) (width 0.2) (layer "F.Cu") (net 4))
 (segment (start 225.8915 89.2868) (end 221.5155 89.2868) (width 0.2) (layer "F.Cu") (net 4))
 (segment (start 196.04 91.46) (end 194.8 92.7) (width 0.2) (layer "F.Cu") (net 4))
 (segment (start 189.64 92.7) (end 185.7 88.76) (width 0.2) (layer "F.Cu") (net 4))
 (segment (start 227.9861 90.6714) (end 227.4052 90.0905) (width 0.2) (layer "F.Cu") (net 4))
 (segment (start 225.6417 96.2111) (end 226.5211 95.3317) (width 0.2) (layer "F.Cu") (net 4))
 (segment (start 221.5155 89.2868) (end 219.3423 91.46) (width 0.2) (layer "F.Cu") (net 4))
 (segment (start 196.6069 87.7798) (end 210.3502 87.7798) (width 0.2) (layer "F.Cu") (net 24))
 (segment (start 189.26 88.78) (end 195.6067 88.78) (width 0.2) (layer "F.Cu") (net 24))
 (segment (start 195.6067 88.78) (end 196.6069 87.7798) (width 0.2) (layer "F.Cu") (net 24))
 (segment (start 210.3502 87.7798) (end 218.1 80.03) (width 0.2) (layer "F.Cu") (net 24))
 (segment (start 209.35 86.24) (end 189.26 86.24) (width 0.2) (layer "F.Cu") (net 23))
 (segment (start 218.1 77.49) (end 209.35 86.24) (width 0.2) (layer "F.Cu") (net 23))
 (segment (start 222.845 91.615) (end 222.845 96.865) (width 0.2) (layer "F.Cu") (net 21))
 (segment (start 223.72 90.74) (end 222.845 91.615) (width 0.2) (layer "F.Cu") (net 21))
 (segment (start 222.845 96.865) (end 223.72 97.74) (width 0.2) (layer "F.Cu") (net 21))
 (segment (start 223.745 94.34) (end 224.6651 95.2601) (width 0.2) (layer "F.Cu") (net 20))
 (segment (start 224.6651 95.2601) (end 224.6651 100.0949) (width 0.2) (layer "F.Cu") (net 20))
 (segment (start 224.6651 100.0949) (end 223.72 101.04) (width 0.2) (layer "F.Cu") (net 20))
 (segment (start 189.36 70) (end 185.76 70) (width 0.2) (layer "F.Cu") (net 17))
 (segment (start 216.9294 71.0406) (end 190.4006 71.0406) (width 0.2) (layer "F.Cu") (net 17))
 (segment (start 190.4006 71.0406) (end 189.36 70) (width 0.2) (layer "F.Cu") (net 17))
 (segment (start 218.1 69.87) (end 216.9294 71.0406) (width 0.2) (layer "F.Cu") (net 17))
 (segment (start 219.251 66.179) (end 219.221 66.149) (width 0.2) (layer "F.Cu") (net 18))
 (segment (start 219.251 71.259) (end 219.251 66.179) (width 0.2) (layer "F.Cu") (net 18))
 (segment (start 190.671 66.149) (end 189.36 67.46) (width 0.2) (layer "F.Cu") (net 18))
 (segment (start 218.1 72.41) (end 219.251 71.259) (width 0.2) (layer "F.Cu") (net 18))
 (segment (start 189.36 67.46) (end 185.76 67.46) (width 0.2) (layer "F.Cu") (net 18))
 (segment (start 219.221 66.149) (end 190.671 66.149) (width 0.2) (layer "F.Cu") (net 18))
 (segment (start 221.2484 101.5116) (end 221.72 101.04) (width 0.2) (layer "F.Cu") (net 9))
 (segment (start 196.0398 101.5116) (end 221.2484 101.5116) (width 0.2) (layer "F.Cu") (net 9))
 (via (at 196.0398 101.5116) (size 0.6) (drill 0.3) (layers "F.Cu" "B.Cu") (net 9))
 (segment (start 196.0398 76.1598) (end 196.0398 101.5116) (width 0.2) (layer "B.Cu") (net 9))
 (segment (start 194.8 74.92) (end 196.0398 76.1598) (width 0.2) (layer "B.Cu") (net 9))
 (segment (start 227.3 67.8) (end 224.5204 67.8) (width 0.2) (layer "F.Cu") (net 19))
 (segment (start 221 67.8) (end 224.5204 67.8) (width 0.2) (layer "F.Cu") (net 19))
 (via (at 224.5204 67.8) (size 0.6) (drill 0.3) (layers "F.Cu" "B.Cu") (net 19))
 (segment (start 216.9235 94.7564) (end 217.7982 93.8817) (width 0.2) (layer "B.Cu") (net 19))
 (segment (start 224.5204 87.9773) (end 224.5204 67.8) (width 0.2) (layer "B.Cu") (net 19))
 (segment (start 218.1 102.89) (end 216.9235 101.7135) (width 0.2) (layer "B.Cu") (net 19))
 (segment (start 218.616 93.8817) (end 224.5204 87.9773) (width 0.2) (layer "B.Cu") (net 19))
 (segment (start 216.9235 101.7135) (end 216.9235 94.7564) (width 0.2) (layer "B.Cu") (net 19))
 (segment (start 217.7982 93.8817) (end 218.616 93.8817) (width 0.2) (layer "B.Cu") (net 19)))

